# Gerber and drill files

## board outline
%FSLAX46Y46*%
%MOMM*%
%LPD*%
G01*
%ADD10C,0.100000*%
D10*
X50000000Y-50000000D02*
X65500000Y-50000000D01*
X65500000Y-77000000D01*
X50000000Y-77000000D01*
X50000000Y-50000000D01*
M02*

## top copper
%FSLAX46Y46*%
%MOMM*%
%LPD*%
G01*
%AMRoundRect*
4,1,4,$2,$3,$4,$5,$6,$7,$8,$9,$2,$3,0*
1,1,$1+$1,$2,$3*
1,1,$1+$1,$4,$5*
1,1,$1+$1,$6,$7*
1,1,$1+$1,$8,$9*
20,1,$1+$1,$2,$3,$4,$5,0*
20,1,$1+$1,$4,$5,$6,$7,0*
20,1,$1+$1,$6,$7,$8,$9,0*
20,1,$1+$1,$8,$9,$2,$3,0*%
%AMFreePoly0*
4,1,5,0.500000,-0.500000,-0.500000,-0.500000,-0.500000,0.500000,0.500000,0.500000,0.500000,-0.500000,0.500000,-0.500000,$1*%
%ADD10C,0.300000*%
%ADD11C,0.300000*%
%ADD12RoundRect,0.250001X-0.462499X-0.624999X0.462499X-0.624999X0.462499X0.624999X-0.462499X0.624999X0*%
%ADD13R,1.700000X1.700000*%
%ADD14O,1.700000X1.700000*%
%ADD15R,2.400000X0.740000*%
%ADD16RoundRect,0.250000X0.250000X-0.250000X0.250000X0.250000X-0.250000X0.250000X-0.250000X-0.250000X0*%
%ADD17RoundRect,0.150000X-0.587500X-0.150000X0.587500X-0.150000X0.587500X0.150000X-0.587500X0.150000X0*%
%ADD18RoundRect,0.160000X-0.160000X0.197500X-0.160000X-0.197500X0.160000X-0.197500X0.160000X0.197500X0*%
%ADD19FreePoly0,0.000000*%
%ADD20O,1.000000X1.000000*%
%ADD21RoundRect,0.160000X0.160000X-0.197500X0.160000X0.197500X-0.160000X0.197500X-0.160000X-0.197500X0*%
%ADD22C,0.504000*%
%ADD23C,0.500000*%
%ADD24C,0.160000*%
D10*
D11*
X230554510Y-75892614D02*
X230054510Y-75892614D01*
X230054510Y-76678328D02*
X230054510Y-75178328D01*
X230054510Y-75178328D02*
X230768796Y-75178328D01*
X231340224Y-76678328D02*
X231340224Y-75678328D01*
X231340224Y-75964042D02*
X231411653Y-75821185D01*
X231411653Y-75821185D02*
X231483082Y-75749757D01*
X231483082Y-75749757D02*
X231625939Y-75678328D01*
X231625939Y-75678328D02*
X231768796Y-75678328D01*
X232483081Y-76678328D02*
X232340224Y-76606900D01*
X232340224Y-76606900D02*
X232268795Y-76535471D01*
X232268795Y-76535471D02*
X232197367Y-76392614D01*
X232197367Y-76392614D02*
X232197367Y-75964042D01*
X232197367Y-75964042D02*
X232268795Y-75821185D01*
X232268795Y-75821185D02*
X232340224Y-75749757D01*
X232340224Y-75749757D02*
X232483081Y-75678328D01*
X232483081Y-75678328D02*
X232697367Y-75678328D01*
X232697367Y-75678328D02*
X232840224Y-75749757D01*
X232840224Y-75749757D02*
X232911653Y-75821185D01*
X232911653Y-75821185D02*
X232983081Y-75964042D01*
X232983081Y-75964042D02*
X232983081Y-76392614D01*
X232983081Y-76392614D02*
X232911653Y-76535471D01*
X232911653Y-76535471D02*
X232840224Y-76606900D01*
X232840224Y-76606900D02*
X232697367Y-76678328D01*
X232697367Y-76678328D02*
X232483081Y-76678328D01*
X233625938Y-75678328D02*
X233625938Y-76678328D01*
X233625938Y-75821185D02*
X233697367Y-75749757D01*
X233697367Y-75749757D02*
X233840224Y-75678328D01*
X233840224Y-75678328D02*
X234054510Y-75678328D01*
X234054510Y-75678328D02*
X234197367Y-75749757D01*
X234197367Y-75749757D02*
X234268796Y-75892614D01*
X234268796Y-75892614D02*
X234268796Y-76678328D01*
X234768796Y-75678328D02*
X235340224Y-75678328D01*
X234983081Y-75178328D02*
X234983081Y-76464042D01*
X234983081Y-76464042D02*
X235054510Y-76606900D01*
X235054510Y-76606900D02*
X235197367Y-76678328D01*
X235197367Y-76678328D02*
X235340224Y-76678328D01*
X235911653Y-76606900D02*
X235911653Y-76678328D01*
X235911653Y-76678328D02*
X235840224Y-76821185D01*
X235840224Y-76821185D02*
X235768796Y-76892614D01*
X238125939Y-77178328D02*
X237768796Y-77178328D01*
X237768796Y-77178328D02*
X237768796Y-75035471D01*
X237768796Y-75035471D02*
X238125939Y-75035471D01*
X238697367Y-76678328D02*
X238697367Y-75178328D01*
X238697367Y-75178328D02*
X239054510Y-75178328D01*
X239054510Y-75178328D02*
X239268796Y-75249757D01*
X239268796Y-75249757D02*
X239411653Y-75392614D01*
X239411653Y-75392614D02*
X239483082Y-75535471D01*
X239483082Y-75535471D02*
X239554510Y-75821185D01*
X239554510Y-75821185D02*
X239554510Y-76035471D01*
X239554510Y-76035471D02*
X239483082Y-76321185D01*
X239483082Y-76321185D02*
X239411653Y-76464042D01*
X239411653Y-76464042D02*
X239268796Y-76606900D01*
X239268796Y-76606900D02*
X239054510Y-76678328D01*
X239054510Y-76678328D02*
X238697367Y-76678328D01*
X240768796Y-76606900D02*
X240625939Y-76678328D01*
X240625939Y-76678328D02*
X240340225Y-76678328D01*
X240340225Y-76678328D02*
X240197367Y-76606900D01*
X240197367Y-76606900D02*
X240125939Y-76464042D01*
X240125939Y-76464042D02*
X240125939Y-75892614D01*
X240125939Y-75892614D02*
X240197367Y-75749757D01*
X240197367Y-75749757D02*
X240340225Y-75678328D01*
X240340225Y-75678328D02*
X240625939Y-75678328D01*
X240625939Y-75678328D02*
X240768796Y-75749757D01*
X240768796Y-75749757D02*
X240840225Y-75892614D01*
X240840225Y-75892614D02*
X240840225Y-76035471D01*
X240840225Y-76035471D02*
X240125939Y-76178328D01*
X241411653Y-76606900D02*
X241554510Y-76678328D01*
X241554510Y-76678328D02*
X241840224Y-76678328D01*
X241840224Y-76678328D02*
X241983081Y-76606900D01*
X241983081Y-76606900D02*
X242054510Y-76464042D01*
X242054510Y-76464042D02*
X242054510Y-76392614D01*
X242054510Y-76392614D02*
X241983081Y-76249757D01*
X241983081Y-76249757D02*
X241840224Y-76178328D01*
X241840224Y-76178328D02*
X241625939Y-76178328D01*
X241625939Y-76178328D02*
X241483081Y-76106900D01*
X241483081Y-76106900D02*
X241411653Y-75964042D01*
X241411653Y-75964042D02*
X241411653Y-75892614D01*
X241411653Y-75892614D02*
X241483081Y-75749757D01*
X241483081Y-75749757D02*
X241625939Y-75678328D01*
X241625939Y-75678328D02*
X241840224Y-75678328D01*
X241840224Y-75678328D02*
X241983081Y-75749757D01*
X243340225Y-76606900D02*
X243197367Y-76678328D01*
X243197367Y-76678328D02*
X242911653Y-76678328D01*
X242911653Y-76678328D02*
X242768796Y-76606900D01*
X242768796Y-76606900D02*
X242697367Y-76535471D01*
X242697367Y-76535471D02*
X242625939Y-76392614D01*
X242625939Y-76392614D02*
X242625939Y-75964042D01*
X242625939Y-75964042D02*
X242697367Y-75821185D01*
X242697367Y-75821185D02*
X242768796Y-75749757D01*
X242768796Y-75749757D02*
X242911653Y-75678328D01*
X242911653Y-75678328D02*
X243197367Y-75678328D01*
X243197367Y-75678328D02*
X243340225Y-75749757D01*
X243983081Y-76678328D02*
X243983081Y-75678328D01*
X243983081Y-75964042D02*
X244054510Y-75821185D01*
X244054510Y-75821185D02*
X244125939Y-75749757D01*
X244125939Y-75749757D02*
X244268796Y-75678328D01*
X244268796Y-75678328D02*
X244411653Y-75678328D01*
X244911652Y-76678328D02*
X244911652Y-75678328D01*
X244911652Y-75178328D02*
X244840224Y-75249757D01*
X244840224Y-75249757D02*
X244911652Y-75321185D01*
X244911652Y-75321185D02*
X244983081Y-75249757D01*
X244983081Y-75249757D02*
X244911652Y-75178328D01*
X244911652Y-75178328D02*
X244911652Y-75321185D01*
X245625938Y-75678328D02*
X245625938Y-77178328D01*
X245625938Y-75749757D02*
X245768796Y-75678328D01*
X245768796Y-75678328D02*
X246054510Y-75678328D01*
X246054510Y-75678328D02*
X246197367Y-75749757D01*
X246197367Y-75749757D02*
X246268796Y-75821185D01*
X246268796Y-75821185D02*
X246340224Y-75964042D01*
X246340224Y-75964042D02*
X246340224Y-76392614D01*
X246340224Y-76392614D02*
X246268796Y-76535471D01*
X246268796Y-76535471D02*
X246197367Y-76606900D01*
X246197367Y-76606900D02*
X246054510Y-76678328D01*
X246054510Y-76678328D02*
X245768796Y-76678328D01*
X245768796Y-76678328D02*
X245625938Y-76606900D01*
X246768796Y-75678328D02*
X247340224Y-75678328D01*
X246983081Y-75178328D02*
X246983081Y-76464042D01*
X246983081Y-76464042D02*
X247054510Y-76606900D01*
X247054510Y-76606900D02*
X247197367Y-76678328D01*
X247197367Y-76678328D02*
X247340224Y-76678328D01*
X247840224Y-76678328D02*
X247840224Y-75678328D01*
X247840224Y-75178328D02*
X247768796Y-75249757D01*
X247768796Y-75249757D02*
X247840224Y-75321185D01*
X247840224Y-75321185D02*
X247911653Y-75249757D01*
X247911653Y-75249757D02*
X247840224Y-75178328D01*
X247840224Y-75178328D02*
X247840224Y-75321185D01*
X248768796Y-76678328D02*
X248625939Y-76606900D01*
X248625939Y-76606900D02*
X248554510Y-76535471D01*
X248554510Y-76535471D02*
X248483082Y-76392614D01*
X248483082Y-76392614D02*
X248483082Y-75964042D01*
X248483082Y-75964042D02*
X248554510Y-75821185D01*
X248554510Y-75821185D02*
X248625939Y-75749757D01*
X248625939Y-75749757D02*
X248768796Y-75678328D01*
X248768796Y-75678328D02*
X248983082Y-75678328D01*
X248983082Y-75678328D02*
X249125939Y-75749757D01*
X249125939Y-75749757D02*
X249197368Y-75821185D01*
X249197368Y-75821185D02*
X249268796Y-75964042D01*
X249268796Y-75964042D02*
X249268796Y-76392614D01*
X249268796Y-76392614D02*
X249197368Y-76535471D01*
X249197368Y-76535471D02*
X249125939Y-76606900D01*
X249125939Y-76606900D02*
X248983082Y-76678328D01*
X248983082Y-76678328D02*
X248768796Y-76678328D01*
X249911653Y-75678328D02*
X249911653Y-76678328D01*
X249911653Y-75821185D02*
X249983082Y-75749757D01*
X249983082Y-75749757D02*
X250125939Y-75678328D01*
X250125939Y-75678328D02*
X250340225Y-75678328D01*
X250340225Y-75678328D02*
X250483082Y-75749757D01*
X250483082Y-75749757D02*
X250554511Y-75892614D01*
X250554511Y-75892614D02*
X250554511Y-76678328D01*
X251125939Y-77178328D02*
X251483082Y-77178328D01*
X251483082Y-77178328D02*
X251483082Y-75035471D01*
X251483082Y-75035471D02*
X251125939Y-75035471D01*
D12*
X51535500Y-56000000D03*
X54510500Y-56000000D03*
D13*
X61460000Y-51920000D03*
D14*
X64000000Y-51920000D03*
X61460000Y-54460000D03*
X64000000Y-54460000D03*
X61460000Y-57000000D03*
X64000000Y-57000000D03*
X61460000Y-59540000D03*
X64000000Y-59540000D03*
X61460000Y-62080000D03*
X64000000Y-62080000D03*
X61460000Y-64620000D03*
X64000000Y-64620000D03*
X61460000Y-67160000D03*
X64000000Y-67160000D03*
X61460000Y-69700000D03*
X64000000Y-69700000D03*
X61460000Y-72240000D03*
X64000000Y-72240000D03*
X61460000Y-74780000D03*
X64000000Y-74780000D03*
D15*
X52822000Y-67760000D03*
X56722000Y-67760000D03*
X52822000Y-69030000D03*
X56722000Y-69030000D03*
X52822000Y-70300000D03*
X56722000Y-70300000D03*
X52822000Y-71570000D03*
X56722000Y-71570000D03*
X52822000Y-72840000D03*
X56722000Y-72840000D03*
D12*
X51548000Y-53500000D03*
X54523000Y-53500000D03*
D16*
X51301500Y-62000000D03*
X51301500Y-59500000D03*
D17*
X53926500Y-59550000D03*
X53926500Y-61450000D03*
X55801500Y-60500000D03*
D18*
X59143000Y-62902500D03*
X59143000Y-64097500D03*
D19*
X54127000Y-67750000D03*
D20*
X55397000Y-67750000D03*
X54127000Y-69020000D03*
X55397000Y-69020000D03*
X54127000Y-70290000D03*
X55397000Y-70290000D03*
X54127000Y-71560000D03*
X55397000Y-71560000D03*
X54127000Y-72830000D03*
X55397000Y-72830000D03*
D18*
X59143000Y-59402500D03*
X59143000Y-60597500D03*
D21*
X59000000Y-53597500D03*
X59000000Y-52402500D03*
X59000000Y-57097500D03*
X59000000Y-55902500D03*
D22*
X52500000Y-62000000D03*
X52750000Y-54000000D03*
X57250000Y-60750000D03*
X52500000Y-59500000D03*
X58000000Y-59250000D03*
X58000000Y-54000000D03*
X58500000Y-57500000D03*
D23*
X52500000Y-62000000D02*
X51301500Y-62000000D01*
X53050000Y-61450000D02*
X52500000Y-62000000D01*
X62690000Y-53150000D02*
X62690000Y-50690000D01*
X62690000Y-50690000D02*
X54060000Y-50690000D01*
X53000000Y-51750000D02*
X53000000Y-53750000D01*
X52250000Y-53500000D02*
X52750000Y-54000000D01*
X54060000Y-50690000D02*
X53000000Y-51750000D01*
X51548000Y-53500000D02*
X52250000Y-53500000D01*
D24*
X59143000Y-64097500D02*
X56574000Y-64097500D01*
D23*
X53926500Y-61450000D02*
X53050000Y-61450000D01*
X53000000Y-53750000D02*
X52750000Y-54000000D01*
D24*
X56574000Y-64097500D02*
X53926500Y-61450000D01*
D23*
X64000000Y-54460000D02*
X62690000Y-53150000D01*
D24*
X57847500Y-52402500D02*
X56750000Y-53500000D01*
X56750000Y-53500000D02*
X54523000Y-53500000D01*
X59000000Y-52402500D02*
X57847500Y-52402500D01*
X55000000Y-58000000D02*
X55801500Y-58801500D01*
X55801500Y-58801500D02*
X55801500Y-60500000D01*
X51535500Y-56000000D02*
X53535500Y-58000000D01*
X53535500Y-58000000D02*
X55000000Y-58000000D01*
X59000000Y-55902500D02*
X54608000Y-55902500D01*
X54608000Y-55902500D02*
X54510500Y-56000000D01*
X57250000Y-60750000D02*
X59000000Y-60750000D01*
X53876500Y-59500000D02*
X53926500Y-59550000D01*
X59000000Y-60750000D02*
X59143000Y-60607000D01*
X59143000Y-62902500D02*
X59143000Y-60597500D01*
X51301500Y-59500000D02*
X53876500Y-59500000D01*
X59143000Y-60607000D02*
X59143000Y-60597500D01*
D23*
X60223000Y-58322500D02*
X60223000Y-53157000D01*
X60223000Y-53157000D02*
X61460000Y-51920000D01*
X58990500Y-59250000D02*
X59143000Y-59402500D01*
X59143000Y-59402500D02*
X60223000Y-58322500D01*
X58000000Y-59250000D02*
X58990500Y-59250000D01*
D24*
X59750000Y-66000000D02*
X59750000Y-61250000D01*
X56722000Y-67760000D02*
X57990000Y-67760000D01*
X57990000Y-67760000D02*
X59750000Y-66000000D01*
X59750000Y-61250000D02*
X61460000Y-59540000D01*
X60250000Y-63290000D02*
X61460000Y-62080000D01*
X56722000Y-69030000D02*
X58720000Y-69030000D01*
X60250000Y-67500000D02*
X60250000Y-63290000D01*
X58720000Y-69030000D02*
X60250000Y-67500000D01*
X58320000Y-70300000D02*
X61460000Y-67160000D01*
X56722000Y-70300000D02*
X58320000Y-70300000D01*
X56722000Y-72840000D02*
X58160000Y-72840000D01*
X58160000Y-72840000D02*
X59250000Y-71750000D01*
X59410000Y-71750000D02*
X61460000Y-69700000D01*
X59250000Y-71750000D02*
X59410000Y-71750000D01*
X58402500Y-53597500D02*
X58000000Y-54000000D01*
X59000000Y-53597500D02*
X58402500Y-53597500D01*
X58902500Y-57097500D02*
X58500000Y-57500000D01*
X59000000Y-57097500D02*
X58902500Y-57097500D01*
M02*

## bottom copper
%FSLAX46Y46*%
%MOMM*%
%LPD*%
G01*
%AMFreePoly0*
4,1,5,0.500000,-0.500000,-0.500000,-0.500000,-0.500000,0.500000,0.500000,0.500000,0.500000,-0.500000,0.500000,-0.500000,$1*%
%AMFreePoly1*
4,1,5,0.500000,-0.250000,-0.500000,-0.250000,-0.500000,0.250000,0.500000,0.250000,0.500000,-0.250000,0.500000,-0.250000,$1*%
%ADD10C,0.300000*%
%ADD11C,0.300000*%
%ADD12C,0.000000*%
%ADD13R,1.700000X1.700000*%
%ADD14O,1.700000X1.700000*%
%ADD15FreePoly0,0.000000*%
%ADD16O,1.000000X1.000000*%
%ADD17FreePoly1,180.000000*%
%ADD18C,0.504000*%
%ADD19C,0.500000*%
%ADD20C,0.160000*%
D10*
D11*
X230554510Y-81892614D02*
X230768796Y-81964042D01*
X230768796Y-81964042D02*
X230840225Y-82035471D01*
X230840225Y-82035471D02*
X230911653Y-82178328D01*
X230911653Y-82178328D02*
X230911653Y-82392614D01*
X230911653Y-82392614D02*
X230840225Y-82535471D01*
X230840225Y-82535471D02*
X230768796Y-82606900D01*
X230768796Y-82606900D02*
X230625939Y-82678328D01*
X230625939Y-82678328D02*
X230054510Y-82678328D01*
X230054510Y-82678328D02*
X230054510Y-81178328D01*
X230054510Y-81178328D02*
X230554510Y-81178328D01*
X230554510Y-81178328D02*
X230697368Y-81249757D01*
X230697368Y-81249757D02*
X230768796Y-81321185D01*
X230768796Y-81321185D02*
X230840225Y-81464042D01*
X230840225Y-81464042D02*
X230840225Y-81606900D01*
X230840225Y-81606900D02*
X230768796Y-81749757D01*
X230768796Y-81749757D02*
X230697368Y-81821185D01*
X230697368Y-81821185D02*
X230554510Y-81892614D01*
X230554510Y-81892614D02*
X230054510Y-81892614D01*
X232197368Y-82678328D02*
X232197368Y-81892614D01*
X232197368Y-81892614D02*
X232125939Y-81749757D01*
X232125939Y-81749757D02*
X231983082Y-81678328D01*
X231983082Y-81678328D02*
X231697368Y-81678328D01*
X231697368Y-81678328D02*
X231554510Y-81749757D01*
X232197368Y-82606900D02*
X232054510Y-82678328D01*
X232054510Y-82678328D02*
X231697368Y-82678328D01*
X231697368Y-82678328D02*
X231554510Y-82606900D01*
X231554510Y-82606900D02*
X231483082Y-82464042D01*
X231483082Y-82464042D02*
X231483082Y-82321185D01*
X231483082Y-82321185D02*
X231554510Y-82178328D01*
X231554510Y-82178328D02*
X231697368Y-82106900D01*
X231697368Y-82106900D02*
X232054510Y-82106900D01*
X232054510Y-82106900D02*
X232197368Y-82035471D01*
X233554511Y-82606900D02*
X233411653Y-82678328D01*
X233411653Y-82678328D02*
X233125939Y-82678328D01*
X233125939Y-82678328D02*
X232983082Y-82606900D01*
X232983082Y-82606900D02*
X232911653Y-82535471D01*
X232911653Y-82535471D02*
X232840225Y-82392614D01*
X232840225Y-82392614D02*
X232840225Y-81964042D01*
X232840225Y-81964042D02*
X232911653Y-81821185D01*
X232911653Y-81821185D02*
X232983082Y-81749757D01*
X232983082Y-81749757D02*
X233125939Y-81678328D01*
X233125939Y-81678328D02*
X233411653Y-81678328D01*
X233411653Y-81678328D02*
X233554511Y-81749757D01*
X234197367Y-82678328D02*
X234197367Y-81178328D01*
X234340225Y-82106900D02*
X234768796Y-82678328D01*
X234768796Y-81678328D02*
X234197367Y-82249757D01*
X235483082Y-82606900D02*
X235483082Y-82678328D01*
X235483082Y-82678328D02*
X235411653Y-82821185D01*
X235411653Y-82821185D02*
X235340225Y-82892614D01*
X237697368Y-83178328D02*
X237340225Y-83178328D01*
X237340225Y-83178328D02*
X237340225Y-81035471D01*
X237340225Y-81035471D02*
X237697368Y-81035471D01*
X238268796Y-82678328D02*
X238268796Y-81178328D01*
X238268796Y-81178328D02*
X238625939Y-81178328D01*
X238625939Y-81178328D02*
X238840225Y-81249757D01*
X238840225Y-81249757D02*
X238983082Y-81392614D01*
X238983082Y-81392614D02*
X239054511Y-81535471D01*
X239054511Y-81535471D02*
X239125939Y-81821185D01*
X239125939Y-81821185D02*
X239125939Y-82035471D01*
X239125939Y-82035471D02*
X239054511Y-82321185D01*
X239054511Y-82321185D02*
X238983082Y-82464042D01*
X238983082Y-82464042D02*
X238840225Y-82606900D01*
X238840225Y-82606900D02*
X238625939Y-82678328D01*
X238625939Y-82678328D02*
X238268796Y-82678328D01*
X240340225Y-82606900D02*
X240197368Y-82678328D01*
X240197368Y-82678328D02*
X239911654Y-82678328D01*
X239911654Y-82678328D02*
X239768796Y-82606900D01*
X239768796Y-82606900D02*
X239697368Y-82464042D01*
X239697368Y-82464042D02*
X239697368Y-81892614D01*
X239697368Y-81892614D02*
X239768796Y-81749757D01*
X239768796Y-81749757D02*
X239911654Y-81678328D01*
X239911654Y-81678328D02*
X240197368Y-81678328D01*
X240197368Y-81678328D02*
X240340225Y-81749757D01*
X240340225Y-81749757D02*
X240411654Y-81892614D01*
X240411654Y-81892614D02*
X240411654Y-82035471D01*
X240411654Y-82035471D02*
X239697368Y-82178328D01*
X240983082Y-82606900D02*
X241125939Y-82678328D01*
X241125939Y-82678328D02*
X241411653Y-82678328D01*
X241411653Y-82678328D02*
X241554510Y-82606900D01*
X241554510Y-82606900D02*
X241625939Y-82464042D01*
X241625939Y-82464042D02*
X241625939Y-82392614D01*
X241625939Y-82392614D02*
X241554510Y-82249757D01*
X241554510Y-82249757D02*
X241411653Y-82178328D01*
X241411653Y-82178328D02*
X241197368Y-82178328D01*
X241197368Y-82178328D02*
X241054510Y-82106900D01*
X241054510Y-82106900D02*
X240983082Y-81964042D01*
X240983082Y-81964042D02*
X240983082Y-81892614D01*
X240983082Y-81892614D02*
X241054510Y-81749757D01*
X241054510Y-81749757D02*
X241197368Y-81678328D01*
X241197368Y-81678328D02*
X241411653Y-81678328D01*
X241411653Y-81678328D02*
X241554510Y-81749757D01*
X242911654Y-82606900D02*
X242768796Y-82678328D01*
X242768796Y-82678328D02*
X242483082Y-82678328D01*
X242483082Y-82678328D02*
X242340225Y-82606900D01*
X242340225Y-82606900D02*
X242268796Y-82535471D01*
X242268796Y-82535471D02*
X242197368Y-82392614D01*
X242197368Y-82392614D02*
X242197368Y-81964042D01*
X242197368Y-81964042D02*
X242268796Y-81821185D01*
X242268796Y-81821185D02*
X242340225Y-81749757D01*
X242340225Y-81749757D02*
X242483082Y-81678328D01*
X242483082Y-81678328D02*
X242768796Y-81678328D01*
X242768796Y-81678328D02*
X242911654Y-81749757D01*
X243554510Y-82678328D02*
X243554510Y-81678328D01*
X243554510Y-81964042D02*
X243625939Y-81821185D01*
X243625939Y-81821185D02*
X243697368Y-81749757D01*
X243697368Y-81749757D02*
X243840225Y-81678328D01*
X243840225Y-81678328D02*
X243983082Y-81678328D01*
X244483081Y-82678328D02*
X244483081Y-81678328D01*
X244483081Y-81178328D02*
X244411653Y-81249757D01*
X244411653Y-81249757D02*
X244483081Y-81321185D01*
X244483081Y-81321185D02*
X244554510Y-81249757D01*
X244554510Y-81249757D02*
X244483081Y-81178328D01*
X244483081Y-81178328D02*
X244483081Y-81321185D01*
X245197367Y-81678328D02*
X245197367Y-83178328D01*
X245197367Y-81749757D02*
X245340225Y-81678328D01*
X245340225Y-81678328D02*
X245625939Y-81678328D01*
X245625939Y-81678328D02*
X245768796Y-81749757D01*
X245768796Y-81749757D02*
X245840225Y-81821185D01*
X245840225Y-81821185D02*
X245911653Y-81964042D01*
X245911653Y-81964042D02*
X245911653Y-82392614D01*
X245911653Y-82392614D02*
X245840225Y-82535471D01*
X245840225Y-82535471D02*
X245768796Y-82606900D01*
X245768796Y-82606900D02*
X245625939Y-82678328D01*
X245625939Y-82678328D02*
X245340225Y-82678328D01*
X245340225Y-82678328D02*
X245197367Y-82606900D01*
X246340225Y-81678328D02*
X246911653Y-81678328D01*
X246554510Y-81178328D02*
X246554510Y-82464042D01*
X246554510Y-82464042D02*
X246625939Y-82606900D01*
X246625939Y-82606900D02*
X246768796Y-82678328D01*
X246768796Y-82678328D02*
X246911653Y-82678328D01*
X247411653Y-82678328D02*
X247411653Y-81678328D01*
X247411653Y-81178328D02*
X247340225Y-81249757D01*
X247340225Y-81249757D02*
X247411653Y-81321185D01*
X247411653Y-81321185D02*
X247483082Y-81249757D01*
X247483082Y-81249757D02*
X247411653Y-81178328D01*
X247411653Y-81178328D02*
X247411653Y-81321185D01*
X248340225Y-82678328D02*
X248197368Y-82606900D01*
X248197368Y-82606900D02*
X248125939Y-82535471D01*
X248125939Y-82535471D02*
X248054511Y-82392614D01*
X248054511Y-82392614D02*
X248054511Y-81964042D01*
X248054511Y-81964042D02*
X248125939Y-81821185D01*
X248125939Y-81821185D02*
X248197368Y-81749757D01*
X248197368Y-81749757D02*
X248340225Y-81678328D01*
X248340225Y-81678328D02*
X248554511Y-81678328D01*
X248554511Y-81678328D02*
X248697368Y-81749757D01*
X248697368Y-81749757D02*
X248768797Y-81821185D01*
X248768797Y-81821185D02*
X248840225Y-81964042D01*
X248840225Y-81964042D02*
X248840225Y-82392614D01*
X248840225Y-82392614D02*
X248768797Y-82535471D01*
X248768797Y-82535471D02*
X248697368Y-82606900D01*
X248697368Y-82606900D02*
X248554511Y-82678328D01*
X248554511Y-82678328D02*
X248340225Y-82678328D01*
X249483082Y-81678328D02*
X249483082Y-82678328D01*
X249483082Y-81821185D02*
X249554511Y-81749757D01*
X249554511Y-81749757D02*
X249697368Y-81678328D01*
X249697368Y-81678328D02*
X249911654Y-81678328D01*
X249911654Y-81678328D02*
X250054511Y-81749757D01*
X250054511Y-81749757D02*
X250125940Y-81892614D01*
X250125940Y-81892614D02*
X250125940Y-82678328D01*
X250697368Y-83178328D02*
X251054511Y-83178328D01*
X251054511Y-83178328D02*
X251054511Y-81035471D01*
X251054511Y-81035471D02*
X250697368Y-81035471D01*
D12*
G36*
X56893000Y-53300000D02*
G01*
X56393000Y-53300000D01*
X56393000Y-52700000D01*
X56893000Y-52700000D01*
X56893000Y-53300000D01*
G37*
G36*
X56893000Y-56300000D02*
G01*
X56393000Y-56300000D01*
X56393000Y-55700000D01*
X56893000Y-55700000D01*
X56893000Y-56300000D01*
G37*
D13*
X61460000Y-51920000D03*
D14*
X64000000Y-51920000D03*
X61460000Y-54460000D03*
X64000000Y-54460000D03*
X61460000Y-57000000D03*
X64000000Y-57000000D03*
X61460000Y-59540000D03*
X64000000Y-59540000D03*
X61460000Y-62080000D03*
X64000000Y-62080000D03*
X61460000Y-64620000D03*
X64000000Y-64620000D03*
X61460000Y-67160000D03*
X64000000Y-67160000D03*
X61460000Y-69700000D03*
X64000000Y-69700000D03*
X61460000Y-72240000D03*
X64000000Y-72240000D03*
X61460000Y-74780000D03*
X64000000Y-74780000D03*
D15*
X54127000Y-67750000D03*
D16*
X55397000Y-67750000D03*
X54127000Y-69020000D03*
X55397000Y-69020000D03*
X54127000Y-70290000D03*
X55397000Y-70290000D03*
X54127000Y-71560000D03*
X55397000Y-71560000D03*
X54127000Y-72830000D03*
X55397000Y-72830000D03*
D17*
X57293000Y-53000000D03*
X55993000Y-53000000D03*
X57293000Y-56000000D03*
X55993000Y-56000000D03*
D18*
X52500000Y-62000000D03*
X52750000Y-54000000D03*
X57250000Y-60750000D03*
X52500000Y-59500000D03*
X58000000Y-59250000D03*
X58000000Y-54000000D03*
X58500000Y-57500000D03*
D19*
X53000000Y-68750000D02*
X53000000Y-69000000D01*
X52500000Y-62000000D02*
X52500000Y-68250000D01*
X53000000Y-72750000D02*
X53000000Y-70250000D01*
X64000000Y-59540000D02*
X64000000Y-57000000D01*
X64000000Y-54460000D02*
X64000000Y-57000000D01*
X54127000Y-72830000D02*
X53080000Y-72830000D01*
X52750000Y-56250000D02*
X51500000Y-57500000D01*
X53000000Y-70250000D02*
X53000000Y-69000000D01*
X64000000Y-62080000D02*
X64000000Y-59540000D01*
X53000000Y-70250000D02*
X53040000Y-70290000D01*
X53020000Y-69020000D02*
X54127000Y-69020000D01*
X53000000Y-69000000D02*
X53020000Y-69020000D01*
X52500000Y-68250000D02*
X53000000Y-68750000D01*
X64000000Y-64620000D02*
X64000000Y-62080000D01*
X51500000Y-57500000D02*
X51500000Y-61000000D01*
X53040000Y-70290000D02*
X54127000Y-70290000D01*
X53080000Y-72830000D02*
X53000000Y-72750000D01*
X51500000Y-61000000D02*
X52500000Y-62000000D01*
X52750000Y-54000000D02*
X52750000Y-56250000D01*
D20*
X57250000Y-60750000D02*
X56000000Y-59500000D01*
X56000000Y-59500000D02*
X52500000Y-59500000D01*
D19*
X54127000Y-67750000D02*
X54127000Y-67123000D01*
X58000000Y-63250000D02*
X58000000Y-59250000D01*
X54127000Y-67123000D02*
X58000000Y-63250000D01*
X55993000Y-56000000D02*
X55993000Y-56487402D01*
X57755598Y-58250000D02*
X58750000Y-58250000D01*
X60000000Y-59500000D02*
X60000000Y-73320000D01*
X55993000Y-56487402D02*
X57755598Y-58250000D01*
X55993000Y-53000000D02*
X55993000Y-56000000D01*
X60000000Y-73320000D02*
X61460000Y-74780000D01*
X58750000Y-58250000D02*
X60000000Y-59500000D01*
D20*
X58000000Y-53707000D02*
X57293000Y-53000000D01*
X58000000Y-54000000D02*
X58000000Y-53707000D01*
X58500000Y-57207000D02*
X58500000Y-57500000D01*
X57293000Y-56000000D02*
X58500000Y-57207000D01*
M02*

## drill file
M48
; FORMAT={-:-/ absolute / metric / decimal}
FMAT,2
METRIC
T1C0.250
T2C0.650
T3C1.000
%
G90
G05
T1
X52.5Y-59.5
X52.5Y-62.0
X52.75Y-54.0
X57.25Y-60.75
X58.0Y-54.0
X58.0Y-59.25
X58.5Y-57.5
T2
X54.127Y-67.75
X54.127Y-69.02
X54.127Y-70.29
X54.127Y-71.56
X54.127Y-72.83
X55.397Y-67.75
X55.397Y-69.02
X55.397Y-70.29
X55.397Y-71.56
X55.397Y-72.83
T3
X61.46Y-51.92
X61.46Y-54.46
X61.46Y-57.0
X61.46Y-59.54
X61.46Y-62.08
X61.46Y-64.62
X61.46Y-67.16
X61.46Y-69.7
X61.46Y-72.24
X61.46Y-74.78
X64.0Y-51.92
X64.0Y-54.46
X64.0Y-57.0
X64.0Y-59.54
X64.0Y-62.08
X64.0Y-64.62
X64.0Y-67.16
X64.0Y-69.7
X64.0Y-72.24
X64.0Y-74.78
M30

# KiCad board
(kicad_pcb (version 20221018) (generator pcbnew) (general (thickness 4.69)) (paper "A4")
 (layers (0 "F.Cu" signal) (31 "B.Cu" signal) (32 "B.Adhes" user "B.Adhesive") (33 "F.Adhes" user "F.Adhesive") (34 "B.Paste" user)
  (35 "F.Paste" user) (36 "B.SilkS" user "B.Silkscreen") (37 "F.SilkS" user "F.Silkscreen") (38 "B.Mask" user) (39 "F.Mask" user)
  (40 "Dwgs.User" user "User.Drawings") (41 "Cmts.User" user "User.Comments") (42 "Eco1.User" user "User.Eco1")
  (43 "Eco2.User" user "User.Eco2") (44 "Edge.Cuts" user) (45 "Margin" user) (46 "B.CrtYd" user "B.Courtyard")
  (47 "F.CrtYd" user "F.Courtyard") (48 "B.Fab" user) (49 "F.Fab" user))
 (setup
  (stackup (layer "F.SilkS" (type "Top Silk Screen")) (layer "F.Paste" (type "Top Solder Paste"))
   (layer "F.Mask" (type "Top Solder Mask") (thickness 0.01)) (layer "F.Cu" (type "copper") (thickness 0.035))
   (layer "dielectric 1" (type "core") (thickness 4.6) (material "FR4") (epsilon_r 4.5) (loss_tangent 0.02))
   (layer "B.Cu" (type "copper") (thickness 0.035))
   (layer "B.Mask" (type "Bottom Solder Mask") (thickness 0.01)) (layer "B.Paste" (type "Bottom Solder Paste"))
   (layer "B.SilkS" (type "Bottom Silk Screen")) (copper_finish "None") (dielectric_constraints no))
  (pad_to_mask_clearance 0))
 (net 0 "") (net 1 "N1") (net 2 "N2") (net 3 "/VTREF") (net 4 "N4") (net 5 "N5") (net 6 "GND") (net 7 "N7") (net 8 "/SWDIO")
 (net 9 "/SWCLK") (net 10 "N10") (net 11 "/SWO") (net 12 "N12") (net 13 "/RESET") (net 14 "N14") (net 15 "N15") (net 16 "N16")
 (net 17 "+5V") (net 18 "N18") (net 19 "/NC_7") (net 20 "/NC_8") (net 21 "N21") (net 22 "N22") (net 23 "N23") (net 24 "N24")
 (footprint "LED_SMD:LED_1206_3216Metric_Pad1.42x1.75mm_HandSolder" (layer "F.Cu") (at 53.023 56)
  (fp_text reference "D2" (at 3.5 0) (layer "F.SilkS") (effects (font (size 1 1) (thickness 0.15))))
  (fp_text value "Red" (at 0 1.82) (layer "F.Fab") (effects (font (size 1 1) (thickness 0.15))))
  (pad "1" smd roundrect (at -1.4875 0) (size 1.425 1.75) (layers "F.Cu" "F.Paste" "F.Mask") (roundrect_rratio 0.175439) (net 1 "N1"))
  (pad "2" smd roundrect (at 1.4875 0) (size 1.425 1.75) (layers "F.Cu" "F.Paste" "F.Mask") (roundrect_rratio 0.175439) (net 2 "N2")))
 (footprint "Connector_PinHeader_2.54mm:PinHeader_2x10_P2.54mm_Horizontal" (layer "F.Cu") (at 61.46 51.92)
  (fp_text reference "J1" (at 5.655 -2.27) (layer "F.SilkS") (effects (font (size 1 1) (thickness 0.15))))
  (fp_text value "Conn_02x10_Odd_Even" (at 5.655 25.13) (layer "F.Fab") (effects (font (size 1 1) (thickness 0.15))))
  (pad "1" thru_hole rect (at 0 0) (size 1.7 1.7) (drill 1) (layers "*.Cu" "*.Mask") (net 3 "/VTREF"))
  (pad "2" thru_hole oval (at 2.54 0) (size 1.7 1.7) (drill 1) (layers "*.Cu" "*.Mask") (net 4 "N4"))
  (pad "3" thru_hole oval (at 0 2.54) (size 1.7 1.7) (drill 1) (layers "*.Cu" "*.Mask") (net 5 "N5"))
  (pad "4" thru_hole oval (at 2.54 2.54) (size 1.7 1.7) (drill 1) (layers "*.Cu" "*.Mask") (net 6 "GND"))
  (pad "5" thru_hole oval (at 0 5.08) (size 1.7 1.7) (drill 1) (layers "*.Cu" "*.Mask") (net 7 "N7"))
  (pad "6" thru_hole oval (at 2.54 5.08) (size 1.7 1.7) (drill 1) (layers "*.Cu" "*.Mask") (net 6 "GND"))
  (pad "7" thru_hole oval (at 0 7.62) (size 1.7 1.7) (drill 1) (layers "*.Cu" "*.Mask") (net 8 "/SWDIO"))
  (pad "8" thru_hole oval (at 2.54 7.62) (size 1.7 1.7) (drill 1) (layers "*.Cu" "*.Mask") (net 6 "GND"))
  (pad "9" thru_hole oval (at 0 10.16) (size 1.7 1.7) (drill 1) (layers "*.Cu" "*.Mask") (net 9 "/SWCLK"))
  (pad "10" thru_hole oval (at 2.54 10.16) (size 1.7 1.7) (drill 1) (layers "*.Cu" "*.Mask") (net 6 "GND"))
  (pad "11" thru_hole oval (at 0 12.7) (size 1.7 1.7) (drill 1) (layers "*.Cu" "*.Mask") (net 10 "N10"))
  (pad "12" thru_hole oval (at 2.54 12.7) (size 1.7 1.7) (drill 1) (layers "*.Cu" "*.Mask") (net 6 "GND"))
  (pad "13" thru_hole oval (at 0 15.24) (size 1.7 1.7) (drill 1) (layers "*.Cu" "*.Mask") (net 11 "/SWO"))
  (pad "14" thru_hole oval (at 2.54 15.24) (size 1.7 1.7) (drill 1) (layers "*.Cu" "*.Mask") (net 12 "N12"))
  (pad "15" thru_hole oval (at 0 17.78) (size 1.7 1.7) (drill 1) (layers "*.Cu" "*.Mask") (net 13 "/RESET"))
  (pad "16" thru_hole oval (at 2.54 17.78) (size 1.7 1.7) (drill 1) (layers "*.Cu" "*.Mask") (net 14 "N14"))
  (pad "17" thru_hole oval (at 0 20.32) (size 1.7 1.7) (drill 1) (layers "*.Cu" "*.Mask") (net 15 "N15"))
  (pad "18" thru_hole oval (at 2.54 20.32) (size 1.7 1.7) (drill 1) (layers "*.Cu" "*.Mask") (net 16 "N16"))
  (pad "19" thru_hole oval (at 0 22.86) (size 1.7 1.7) (drill 1) (layers "*.Cu" "*.Mask") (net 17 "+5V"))
  (pad "20" thru_hole oval (at 2.54 22.86) (size 1.7 1.7) (drill 1) (layers "*.Cu" "*.Mask") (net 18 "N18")))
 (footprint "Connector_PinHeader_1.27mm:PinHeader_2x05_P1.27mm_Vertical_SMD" (layer "F.Cu") (at 54.772 70.3)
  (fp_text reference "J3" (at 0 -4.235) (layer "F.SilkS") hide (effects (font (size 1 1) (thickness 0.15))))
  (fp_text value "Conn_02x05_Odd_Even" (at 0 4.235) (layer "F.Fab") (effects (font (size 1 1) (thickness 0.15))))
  (pad "1" smd rect (at -1.95 -2.54) (size 2.4 0.74) (layers "F.Cu" "F.Paste" "F.Mask") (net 3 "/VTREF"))
  (pad "2" smd rect (at 1.95 -2.54) (size 2.4 0.74) (layers "F.Cu" "F.Paste" "F.Mask") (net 8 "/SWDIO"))
  (pad "3" smd rect (at -1.95 -1.27) (size 2.4 0.74) (layers "F.Cu" "F.Paste" "F.Mask") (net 6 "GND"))
  (pad "4" smd rect (at 1.95 -1.27) (size 2.4 0.74) (layers "F.Cu" "F.Paste" "F.Mask") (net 9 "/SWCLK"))
  (pad "5" smd rect (at -1.95 0) (size 2.4 0.74) (layers "F.Cu" "F.Paste" "F.Mask") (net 6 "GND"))
  (pad "6" smd rect (at 1.95 0) (size 2.4 0.74) (layers "F.Cu" "F.Paste" "F.Mask") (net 11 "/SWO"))
  (pad "7" smd rect (at -1.95 1.27) (size 2.4 0.74) (layers "F.Cu" "F.Paste" "F.Mask") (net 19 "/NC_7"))
  (pad "8" smd rect (at 1.95 1.27) (size 2.4 0.74) (layers "F.Cu" "F.Paste" "F.Mask") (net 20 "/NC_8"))
  (pad "9" smd rect (at -1.95 2.54) (size 2.4 0.74) (layers "F.Cu" "F.Paste" "F.Mask") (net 6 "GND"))
  (pad "10" smd rect (at 1.95 2.54) (size 2.4 0.74) (layers "F.Cu" "F.Paste" "F.Mask") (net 13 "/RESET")))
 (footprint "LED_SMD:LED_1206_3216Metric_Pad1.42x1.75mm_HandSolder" (layer "F.Cu") (at 53.0355 53.5)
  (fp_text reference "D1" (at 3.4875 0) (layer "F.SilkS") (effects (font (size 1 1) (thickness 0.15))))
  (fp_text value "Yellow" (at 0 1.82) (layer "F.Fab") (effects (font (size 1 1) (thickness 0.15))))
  (pad "1" smd roundrect (at -1.4875 0) (size 1.425 1.75) (layers "F.Cu" "F.Paste" "F.Mask") (roundrect_rratio 0.175439) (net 6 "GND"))
  (pad "2" smd roundrect (at 1.4875 0) (size 1.425 1.75) (layers "F.Cu" "F.Paste" "F.Mask") (roundrect_rratio 0.175439) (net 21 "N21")))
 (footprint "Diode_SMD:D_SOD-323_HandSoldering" (layer "F.Cu") (at 51.3015 60.75 90)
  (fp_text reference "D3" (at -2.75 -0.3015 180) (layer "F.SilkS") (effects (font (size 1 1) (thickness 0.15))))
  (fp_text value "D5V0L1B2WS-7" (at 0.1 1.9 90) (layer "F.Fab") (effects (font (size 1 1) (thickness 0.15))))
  (pad "1" smd roundrect (at -1.25 0 90) (size 1 1) (layers "F.Cu" "F.Paste" "F.Mask") (roundrect_rratio 0.25) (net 6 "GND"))
  (pad "2" smd roundrect (at 1.25 0 90) (size 1 1) (layers "F.Cu" "F.Paste" "F.Mask") (roundrect_rratio 0.25) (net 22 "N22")))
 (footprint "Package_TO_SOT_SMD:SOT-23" (layer "F.Cu") (at 54.864 60.5)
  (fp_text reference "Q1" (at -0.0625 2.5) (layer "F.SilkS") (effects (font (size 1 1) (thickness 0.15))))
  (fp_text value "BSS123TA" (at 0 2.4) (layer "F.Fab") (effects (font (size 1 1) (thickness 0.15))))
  (pad "1" smd roundrect (at -0.9375 -0.95) (size 1.475 0.6) (layers "F.Cu" "F.Paste" "F.Mask") (roundrect_rratio 0.25) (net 22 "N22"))
  (pad "2" smd roundrect (at -0.9375 0.95) (size 1.475 0.6) (layers "F.Cu" "F.Paste" "F.Mask") (roundrect_rratio 0.25) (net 6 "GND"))
  (pad "3" smd roundrect (at 0.9375 0) (size 1.475 0.6) (layers "F.Cu" "F.Paste" "F.Mask") (roundrect_rratio 0.25) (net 1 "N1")))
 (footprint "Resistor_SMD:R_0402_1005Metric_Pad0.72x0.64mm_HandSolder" (layer "F.Cu") (at 59.143 63.5 -90)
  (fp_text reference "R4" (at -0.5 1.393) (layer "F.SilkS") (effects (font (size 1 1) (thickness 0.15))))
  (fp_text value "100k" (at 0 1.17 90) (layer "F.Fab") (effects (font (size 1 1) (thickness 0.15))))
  (pad "1" smd roundrect (at -0.5975 0 270) (size 0.715 0.64) (layers "F.Cu" "F.Paste" "F.Mask") (roundrect_rratio 0.25) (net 22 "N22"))
  (pad "2" smd roundrect (at 0.5975 0 270) (size 0.715 0.64) (layers "F.Cu" "F.Paste" "F.Mask") (roundrect_rratio 0.25) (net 6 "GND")))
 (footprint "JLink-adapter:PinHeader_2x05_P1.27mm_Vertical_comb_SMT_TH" (layer "F.Cu") (at 54.127 67.75)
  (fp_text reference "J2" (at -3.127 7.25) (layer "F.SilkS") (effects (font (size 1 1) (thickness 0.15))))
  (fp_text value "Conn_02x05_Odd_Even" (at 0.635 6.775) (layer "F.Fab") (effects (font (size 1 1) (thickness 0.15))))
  (pad "1" thru_hole custom (at 0 0) (size 1 1) (drill 0.65) (layers "*.Cu" "*.Mask") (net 3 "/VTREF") (thermal_bridge_angle 45)
   (options (clearance outline) (anchor rect)) (primitives))
  (pad "2" thru_hole oval (at 1.27 0) (size 1 1) (drill 0.65) (layers "*.Cu" "*.Mask") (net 8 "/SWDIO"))
  (pad "3" thru_hole oval (at 0 1.27) (size 1 1) (drill 0.65) (layers "*.Cu" "*.Mask") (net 6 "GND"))
  (pad "4" thru_hole oval (at 1.27 1.27) (size 1 1) (drill 0.65) (layers "*.Cu" "*.Mask") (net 9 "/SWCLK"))
  (pad "5" thru_hole oval (at 0 2.54) (size 1 1) (drill 0.65) (layers "*.Cu" "*.Mask") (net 6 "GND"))
  (pad "6" thru_hole oval (at 1.27 2.54) (size 1 1) (drill 0.65) (layers "*.Cu" "*.Mask") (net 11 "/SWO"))
  (pad "7" thru_hole oval (at 0 3.81) (size 1 1) (drill 0.65) (layers "*.Cu" "*.Mask") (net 19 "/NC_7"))
  (pad "8" thru_hole oval (at 1.27 3.81) (size 1 1) (drill 0.65) (layers "*.Cu" "*.Mask") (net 20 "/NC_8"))
  (pad "9" thru_hole oval (at 0 5.08) (size 1 1) (drill 0.65) (layers "*.Cu" "*.Mask") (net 6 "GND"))
  (pad "10" thru_hole oval (at 1.27 5.08) (size 1 1) (drill 0.65) (layers "*.Cu" "*.Mask") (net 13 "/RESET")))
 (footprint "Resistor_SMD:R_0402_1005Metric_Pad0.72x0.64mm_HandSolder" (layer "F.Cu") (at 59.143 60 -90)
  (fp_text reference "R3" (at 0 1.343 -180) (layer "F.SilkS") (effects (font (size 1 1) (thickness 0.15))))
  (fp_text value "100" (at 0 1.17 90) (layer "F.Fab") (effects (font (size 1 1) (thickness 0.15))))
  (pad "1" smd roundrect (at -0.5975 0 270) (size 0.715 0.64) (layers "F.Cu" "F.Paste" "F.Mask") (roundrect_rratio 0.25) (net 3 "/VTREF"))
  (pad "2" smd roundrect (at 0.5975 0 270) (size 0.715 0.64) (layers "F.Cu" "F.Paste" "F.Mask") (roundrect_rratio 0.25) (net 22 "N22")))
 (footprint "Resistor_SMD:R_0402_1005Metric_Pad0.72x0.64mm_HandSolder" (layer "F.Cu") (at 59 53 90)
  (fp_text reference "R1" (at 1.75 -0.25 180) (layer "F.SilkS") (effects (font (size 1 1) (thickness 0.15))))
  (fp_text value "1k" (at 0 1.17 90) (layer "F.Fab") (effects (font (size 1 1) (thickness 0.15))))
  (pad "1" smd roundrect (at -0.5975 0 90) (size 0.715 0.64) (layers "F.Cu" "F.Paste" "F.Mask") (roundrect_rratio 0.25) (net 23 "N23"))
  (pad "2" smd roundrect (at 0.5975 0 90) (size 0.715 0.64) (layers "F.Cu" "F.Paste" "F.Mask") (roundrect_rratio 0.25) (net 21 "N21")))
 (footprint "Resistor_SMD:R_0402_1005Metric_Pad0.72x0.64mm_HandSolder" (layer "F.Cu") (at 59 56.5 90)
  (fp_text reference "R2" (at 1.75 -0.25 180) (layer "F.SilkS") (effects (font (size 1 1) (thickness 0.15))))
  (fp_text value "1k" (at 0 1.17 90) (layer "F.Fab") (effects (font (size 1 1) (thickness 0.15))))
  (pad "1" smd roundrect (at -0.5975 0 90) (size 0.715 0.64) (layers "F.Cu" "F.Paste" "F.Mask") (roundrect_rratio 0.25) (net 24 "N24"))
  (pad "2" smd roundrect (at 0.5975 0 90) (size 0.715 0.64) (layers "F.Cu" "F.Paste" "F.Mask") (roundrect_rratio 0.25) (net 2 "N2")))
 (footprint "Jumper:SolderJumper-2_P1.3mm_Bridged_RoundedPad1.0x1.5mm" (layer "B.Cu") (at 56.643 53 180) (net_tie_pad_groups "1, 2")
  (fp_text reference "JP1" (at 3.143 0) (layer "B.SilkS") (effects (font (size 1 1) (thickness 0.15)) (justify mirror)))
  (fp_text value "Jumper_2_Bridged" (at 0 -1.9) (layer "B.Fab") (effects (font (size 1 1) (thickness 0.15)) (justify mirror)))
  (fp_poly (pts (xy 0.25 0.3) (xy -0.25 0.3) (xy -0.25 -0.3) (xy 0.25 -0.3)) (stroke (width 0) (type solid)) (fill solid) (layer "B.Cu"))
  (pad "1" smd custom (at -0.65 0 180) (size 1 0.5) (layers "B.Cu" "B.Mask") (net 23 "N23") (zone_connect 2) (thermal_bridge_angle 45)
   (options (clearance outline) (anchor rect)) (primitives))
  (pad "2" smd custom (at 0.65 0 180) (size 1 0.5) (layers "B.Cu" "B.Mask") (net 17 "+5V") (zone_connect 2) (thermal_bridge_angle 45)
   (options (clearance outline) (anchor rect)) (primitives)))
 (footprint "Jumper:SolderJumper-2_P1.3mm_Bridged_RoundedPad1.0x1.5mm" (layer "B.Cu") (at 56.643 56 180) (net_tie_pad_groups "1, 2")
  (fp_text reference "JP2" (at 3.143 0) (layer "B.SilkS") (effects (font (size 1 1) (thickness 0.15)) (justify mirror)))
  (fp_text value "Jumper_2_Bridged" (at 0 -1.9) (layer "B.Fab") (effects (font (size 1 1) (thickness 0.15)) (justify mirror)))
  (fp_poly (pts (xy 0.25 0.3) (xy -0.25 0.3) (xy -0.25 -0.3) (xy 0.25 -0.3)) (stroke (width 0) (type solid)) (fill solid) (layer "B.Cu"))
  (pad "1" smd custom (at -0.65 0 180) (size 1 0.5) (layers "B.Cu" "B.Mask") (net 24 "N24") (zone_connect 2) (thermal_bridge_angle 45)
   (options (clearance outline) (anchor rect)) (primitives))
  (pad "2" smd custom (at 0.65 0 180) (size 1 0.5) (layers "B.Cu" "B.Mask") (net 17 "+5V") (zone_connect 2) (thermal_bridge_angle 45)
   (options (clearance outline) (anchor rect)) (primitives)))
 (gr_rect (start 50 50) (end 65.5 77) (stroke (width 0.1) (type default)) (fill none) (layer "Edge.Cuts"))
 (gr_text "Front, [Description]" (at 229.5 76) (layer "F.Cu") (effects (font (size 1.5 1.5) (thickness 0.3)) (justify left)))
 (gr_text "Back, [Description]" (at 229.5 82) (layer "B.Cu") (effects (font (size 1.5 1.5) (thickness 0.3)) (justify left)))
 (segment (start 52.5 62) (end 51.3015 62) (width 0.5) (layer "F.Cu") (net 6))
 (segment (start 53.05 61.45) (end 52.5 62) (width 0.5) (layer "F.Cu") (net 6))
 (segment (start 62.69 53.15) (end 62.69 50.69) (width 0.5) (layer "F.Cu") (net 6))
 (segment (start 62.69 50.69) (end 54.06 50.69) (width 0.5) (layer "F.Cu") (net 6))
 (segment (start 53 51.75) (end 53 53.75) (width 0.5) (layer "F.Cu") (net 6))
 (segment (start 52.25 53.5) (end 52.75 54) (width 0.5) (layer "F.Cu") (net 6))
 (segment (start 54.06 50.69) (end 53 51.75) (width 0.5) (layer "F.Cu") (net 6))
 (segment (start 51.548 53.5) (end 52.25 53.5) (width 0.5) (layer "F.Cu") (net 6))
 (segment (start 59.143 64.0975) (end 56.574 64.0975) (width 0.16) (layer "F.Cu") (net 6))
 (segment (start 53.9265 61.45) (end 53.05 61.45) (width 0.5) (layer "F.Cu") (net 6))
 (segment (start 53 53.75) (end 52.75 54) (width 0.5) (layer "F.Cu") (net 6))
 (segment (start 56.574 64.0975) (end 53.9265 61.45) (width 0.16) (layer "F.Cu") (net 6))
 (segment (start 64 54.46) (end 62.69 53.15) (width 0.5) (layer "F.Cu") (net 6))
 (via (at 52.5 62) (size 0.504) (drill 0.25) (layers "F.Cu" "B.Cu") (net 6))
 (via (at 52.75 54) (size 0.504) (drill 0.25) (layers "F.Cu" "B.Cu") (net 6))
 (segment (start 53 68.75) (end 53 69) (width 0.5) (layer "B.Cu") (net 6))
 (segment (start 52.5 62) (end 52.5 68.25) (width 0.5) (layer "B.Cu") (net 6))
 (segment (start 53 72.75) (end 53 70.25) (width 0.5) (layer "B.Cu") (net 6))
 (segment (start 64 59.54) (end 64 57) (width 0.5) (layer "B.Cu") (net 6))
 (segment (start 64 54.46) (end 64 57) (width 0.5) (layer "B.Cu") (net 6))
 (segment (start 54.127 72.83) (end 53.08 72.83) (width 0.5) (layer "B.Cu") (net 6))
 (segment (start 52.75 56.25) (end 51.5 57.5) (width 0.5) (layer "B.Cu") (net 6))
 (segment (start 53 70.25) (end 53 69) (width 0.5) (layer "B.Cu") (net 6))
 (segment (start 64 62.08) (end 64 59.54) (width 0.5) (layer "B.Cu") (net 6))
 (segment (start 53 70.25) (end 53.04 70.29) (width 0.5) (layer "B.Cu") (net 6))
 (segment (start 53.02 69.02) (end 54.127 69.02) (width 0.5) (layer "B.Cu") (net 6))
 (segment (start 53 69) (end 53.02 69.02) (width 0.5) (layer "B.Cu") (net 6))
 (segment (start 52.5 68.25) (end 53 68.75) (width 0.5) (layer "B.Cu") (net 6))
 (segment (start 64 64.62) (end 64 62.08) (width 0.5) (layer "B.Cu") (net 6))
 (segment (start 51.5 57.5) (end 51.5 61) (width 0.5) (layer "B.Cu") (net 6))
 (segment (start 53.04 70.29) (end 54.127 70.29) (width 0.5) (layer "B.Cu") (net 6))
 (segment (start 53.08 72.83) (end 53 72.75) (width 0.5) (layer "B.Cu") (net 6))
 (segment (start 51.5 61) (end 52.5 62) (width 0.5) (layer "B.Cu") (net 6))
 (segment (start 52.75 54) (end 52.75 56.25) (width 0.5) (layer "B.Cu") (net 6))
 (segment (start 57.8475 52.4025) (end 56.75 53.5) (width 0.16) (layer "F.Cu") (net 21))
 (segment (start 56.75 53.5) (end 54.523 53.5) (width 0.16) (layer "F.Cu") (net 21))
 (segment (start 59 52.4025) (end 57.8475 52.4025) (width 0.16) (layer "F.Cu") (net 21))
 (segment (start 55 58) (end 55.8015 58.8015) (width 0.16) (layer "F.Cu") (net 1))
 (segment (start 55.8015 58.8015) (end 55.8015 60.5) (width 0.16) (layer "F.Cu") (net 1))
 (segment (start 51.5355 56) (end 53.5355 58) (width 0.16) (layer "F.Cu") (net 1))
 (segment (start 53.5355 58) (end 55 58) (width 0.16) (layer "F.Cu") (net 1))
 (segment (start 59 55.9025) (end 54.608 55.9025) (width 0.16) (layer "F.Cu") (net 2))
 (segment (start 54.608 55.9025) (end 54.5105 56) (width 0.16) (layer "F.Cu") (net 2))
 (segment (start 57.25 60.75) (end 59 60.75) (width 0.16) (layer "F.Cu") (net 22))
 (segment (start 53.8765 59.5) (end 53.9265 59.55) (width 0.16) (layer "F.Cu") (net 22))
 (segment (start 59 60.75) (end 59.143 60.607) (width 0.16) (layer "F.Cu") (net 22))
 (segment (start 59.143 62.9025) (end 59.143 60.5975) (width 0.16) (layer "F.Cu") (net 22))
 (segment (start 51.3015 59.5) (end 53.8765 59.5) (width 0.16) (layer "F.Cu") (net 22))
 (segment (start 59.143 60.607) (end 59.143 60.5975) (width 0.16) (layer "F.Cu") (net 22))
 (via (at 57.25 60.75) (size 0.504) (drill 0.25) (layers "F.Cu" "B.Cu") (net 22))
 (via (at 52.5 59.5) (size 0.504) (drill 0.25) (layers "F.Cu" "B.Cu") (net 22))
 (segment (start 57.25 60.75) (end 56 59.5) (width 0.16) (layer "B.Cu") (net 22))
 (segment (start 56 59.5) (end 52.5 59.5) (width 0.16) (layer "B.Cu") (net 22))
 (segment (start 60.223 58.3225) (end 60.223 53.157) (width 0.5) (layer "F.Cu") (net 3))
 (segment (start 60.223 53.157) (end 61.46 51.92) (width 0.5) (layer "F.Cu") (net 3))
 (segment (start 58.9905 59.25) (end 59.143 59.4025) (width 0.5) (layer "F.Cu") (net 3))
 (segment (start 59.143 59.4025) (end 60.223 58.3225) (width 0.5) (layer "F.Cu") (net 3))
 (segment (start 58 59.25) (end 58.9905 59.25) (width 0.5) (layer "F.Cu") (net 3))
 (via (at 58 59.25) (size 0.504) (drill 0.25) (layers "F.Cu" "B.Cu") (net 3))
 (segment (start 54.127 67.75) (end 54.127 67.123) (width 0.5) (layer "B.Cu") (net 3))
 (segment (start 58 63.25) (end 58 59.25) (width 0.5) (layer "B.Cu") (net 3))
 (segment (start 54.127 67.123) (end 58 63.25) (width 0.5) (layer "B.Cu") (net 3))
 (segment (start 59.75 66) (end 59.75 61.25) (width 0.16) (layer "F.Cu") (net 8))
 (segment (start 56.722 67.76) (end 57.99 67.76) (width 0.16) (layer "F.Cu") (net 8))
 (segment (start 57.99 67.76) (end 59.75 66) (width 0.16) (layer "F.Cu") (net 8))
 (segment (start 59.75 61.25) (end 61.46 59.54) (width 0.16) (layer "F.Cu") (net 8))
 (segment (start 60.25 63.29) (end 61.46 62.08) (width 0.16) (layer "F.Cu") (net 9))
 (segment (start 56.722 69.03) (end 58.72 69.03) (width 0.16) (layer "F.Cu") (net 9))
 (segment (start 60.25 67.5) (end 60.25 63.29) (width 0.16) (layer "F.Cu") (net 9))
 (segment (start 58.72 69.03) (end 60.25 67.5) (width 0.16) (layer "F.Cu") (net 9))
 (segment (start 58.32 70.3) (end 61.46 67.16) (width 0.16) (layer "F.Cu") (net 11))
 (segment (start 56.722 70.3) (end 58.32 70.3) (width 0.16) (layer "F.Cu") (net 11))
 (segment (start 56.722 72.84) (end 58.16 72.84) (width 0.16) (layer "F.Cu") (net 13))
 (segment (start 58.16 72.84) (end 59.25 71.75) (width 0.16) (layer "F.Cu") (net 13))
 (segment (start 59.41 71.75) (end 61.46 69.7) (width 0.16) (layer "F.Cu") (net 13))
 (segment (start 59.25 71.75) (end 59.41 71.75) (width 0.16) (layer "F.Cu") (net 13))
 (segment (start 55.993 56) (end 55.993 56.487402) (width 0.5) (layer "B.Cu") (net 17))
 (segment (start 57.755598 58.25) (end 58.75 58.25) (width 0.5) (layer "B.Cu") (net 17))
 (segment (start 60 59.5) (end 60 73.32) (width 0.5) (layer "B.Cu") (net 17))
 (segment (start 55.993 56.487402) (end 57.755598 58.25) (width 0.5) (layer "B.Cu") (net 17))
 (segment (start 55.993 53) (end 55.993 56) (width 0.5) (layer "B.Cu") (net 17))
 (segment (start 60 73.32) (end 61.46 74.78) (width 0.5) (layer "B.Cu") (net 17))
 (segment (start 58.75 58.25) (end 60 59.5) (width 0.5) (layer "B.Cu") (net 17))
 (segment (start 58.4025 53.5975) (end 58 54) (width 0.16) (layer "F.Cu") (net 23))
 (segment (start 59 53.5975) (end 58.4025 53.5975) (width 0.16) (layer "F.Cu") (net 23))
 (via (at 58 54) (size 0.504) (drill 0.25) (layers "F.Cu" "B.Cu") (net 23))
 (segment (start 58 53.707) (end 57.293 53) (width 0.16) (layer "B.Cu") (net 23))
 (segment (start 58 54) (end 58 53.707) (width 0.16) (layer "B.Cu") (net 23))
 (segment (start 58.9025 57.0975) (end 58.5 57.5) (width 0.16) (layer "F.Cu") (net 24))
 (segment (start 59 57.0975) (end 58.9025 57.0975) (width 0.16) (layer "F.Cu") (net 24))
 (via (at 58.5 57.5) (size 0.504) (drill 0.25) (layers "F.Cu" "B.Cu") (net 24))
 (segment (start 58.5 57.207) (end 58.5 57.5) (width 0.16) (layer "B.Cu") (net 24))
 (segment (start 57.293 56) (end 58.5 57.207) (width 0.16) (layer "B.Cu") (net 24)))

